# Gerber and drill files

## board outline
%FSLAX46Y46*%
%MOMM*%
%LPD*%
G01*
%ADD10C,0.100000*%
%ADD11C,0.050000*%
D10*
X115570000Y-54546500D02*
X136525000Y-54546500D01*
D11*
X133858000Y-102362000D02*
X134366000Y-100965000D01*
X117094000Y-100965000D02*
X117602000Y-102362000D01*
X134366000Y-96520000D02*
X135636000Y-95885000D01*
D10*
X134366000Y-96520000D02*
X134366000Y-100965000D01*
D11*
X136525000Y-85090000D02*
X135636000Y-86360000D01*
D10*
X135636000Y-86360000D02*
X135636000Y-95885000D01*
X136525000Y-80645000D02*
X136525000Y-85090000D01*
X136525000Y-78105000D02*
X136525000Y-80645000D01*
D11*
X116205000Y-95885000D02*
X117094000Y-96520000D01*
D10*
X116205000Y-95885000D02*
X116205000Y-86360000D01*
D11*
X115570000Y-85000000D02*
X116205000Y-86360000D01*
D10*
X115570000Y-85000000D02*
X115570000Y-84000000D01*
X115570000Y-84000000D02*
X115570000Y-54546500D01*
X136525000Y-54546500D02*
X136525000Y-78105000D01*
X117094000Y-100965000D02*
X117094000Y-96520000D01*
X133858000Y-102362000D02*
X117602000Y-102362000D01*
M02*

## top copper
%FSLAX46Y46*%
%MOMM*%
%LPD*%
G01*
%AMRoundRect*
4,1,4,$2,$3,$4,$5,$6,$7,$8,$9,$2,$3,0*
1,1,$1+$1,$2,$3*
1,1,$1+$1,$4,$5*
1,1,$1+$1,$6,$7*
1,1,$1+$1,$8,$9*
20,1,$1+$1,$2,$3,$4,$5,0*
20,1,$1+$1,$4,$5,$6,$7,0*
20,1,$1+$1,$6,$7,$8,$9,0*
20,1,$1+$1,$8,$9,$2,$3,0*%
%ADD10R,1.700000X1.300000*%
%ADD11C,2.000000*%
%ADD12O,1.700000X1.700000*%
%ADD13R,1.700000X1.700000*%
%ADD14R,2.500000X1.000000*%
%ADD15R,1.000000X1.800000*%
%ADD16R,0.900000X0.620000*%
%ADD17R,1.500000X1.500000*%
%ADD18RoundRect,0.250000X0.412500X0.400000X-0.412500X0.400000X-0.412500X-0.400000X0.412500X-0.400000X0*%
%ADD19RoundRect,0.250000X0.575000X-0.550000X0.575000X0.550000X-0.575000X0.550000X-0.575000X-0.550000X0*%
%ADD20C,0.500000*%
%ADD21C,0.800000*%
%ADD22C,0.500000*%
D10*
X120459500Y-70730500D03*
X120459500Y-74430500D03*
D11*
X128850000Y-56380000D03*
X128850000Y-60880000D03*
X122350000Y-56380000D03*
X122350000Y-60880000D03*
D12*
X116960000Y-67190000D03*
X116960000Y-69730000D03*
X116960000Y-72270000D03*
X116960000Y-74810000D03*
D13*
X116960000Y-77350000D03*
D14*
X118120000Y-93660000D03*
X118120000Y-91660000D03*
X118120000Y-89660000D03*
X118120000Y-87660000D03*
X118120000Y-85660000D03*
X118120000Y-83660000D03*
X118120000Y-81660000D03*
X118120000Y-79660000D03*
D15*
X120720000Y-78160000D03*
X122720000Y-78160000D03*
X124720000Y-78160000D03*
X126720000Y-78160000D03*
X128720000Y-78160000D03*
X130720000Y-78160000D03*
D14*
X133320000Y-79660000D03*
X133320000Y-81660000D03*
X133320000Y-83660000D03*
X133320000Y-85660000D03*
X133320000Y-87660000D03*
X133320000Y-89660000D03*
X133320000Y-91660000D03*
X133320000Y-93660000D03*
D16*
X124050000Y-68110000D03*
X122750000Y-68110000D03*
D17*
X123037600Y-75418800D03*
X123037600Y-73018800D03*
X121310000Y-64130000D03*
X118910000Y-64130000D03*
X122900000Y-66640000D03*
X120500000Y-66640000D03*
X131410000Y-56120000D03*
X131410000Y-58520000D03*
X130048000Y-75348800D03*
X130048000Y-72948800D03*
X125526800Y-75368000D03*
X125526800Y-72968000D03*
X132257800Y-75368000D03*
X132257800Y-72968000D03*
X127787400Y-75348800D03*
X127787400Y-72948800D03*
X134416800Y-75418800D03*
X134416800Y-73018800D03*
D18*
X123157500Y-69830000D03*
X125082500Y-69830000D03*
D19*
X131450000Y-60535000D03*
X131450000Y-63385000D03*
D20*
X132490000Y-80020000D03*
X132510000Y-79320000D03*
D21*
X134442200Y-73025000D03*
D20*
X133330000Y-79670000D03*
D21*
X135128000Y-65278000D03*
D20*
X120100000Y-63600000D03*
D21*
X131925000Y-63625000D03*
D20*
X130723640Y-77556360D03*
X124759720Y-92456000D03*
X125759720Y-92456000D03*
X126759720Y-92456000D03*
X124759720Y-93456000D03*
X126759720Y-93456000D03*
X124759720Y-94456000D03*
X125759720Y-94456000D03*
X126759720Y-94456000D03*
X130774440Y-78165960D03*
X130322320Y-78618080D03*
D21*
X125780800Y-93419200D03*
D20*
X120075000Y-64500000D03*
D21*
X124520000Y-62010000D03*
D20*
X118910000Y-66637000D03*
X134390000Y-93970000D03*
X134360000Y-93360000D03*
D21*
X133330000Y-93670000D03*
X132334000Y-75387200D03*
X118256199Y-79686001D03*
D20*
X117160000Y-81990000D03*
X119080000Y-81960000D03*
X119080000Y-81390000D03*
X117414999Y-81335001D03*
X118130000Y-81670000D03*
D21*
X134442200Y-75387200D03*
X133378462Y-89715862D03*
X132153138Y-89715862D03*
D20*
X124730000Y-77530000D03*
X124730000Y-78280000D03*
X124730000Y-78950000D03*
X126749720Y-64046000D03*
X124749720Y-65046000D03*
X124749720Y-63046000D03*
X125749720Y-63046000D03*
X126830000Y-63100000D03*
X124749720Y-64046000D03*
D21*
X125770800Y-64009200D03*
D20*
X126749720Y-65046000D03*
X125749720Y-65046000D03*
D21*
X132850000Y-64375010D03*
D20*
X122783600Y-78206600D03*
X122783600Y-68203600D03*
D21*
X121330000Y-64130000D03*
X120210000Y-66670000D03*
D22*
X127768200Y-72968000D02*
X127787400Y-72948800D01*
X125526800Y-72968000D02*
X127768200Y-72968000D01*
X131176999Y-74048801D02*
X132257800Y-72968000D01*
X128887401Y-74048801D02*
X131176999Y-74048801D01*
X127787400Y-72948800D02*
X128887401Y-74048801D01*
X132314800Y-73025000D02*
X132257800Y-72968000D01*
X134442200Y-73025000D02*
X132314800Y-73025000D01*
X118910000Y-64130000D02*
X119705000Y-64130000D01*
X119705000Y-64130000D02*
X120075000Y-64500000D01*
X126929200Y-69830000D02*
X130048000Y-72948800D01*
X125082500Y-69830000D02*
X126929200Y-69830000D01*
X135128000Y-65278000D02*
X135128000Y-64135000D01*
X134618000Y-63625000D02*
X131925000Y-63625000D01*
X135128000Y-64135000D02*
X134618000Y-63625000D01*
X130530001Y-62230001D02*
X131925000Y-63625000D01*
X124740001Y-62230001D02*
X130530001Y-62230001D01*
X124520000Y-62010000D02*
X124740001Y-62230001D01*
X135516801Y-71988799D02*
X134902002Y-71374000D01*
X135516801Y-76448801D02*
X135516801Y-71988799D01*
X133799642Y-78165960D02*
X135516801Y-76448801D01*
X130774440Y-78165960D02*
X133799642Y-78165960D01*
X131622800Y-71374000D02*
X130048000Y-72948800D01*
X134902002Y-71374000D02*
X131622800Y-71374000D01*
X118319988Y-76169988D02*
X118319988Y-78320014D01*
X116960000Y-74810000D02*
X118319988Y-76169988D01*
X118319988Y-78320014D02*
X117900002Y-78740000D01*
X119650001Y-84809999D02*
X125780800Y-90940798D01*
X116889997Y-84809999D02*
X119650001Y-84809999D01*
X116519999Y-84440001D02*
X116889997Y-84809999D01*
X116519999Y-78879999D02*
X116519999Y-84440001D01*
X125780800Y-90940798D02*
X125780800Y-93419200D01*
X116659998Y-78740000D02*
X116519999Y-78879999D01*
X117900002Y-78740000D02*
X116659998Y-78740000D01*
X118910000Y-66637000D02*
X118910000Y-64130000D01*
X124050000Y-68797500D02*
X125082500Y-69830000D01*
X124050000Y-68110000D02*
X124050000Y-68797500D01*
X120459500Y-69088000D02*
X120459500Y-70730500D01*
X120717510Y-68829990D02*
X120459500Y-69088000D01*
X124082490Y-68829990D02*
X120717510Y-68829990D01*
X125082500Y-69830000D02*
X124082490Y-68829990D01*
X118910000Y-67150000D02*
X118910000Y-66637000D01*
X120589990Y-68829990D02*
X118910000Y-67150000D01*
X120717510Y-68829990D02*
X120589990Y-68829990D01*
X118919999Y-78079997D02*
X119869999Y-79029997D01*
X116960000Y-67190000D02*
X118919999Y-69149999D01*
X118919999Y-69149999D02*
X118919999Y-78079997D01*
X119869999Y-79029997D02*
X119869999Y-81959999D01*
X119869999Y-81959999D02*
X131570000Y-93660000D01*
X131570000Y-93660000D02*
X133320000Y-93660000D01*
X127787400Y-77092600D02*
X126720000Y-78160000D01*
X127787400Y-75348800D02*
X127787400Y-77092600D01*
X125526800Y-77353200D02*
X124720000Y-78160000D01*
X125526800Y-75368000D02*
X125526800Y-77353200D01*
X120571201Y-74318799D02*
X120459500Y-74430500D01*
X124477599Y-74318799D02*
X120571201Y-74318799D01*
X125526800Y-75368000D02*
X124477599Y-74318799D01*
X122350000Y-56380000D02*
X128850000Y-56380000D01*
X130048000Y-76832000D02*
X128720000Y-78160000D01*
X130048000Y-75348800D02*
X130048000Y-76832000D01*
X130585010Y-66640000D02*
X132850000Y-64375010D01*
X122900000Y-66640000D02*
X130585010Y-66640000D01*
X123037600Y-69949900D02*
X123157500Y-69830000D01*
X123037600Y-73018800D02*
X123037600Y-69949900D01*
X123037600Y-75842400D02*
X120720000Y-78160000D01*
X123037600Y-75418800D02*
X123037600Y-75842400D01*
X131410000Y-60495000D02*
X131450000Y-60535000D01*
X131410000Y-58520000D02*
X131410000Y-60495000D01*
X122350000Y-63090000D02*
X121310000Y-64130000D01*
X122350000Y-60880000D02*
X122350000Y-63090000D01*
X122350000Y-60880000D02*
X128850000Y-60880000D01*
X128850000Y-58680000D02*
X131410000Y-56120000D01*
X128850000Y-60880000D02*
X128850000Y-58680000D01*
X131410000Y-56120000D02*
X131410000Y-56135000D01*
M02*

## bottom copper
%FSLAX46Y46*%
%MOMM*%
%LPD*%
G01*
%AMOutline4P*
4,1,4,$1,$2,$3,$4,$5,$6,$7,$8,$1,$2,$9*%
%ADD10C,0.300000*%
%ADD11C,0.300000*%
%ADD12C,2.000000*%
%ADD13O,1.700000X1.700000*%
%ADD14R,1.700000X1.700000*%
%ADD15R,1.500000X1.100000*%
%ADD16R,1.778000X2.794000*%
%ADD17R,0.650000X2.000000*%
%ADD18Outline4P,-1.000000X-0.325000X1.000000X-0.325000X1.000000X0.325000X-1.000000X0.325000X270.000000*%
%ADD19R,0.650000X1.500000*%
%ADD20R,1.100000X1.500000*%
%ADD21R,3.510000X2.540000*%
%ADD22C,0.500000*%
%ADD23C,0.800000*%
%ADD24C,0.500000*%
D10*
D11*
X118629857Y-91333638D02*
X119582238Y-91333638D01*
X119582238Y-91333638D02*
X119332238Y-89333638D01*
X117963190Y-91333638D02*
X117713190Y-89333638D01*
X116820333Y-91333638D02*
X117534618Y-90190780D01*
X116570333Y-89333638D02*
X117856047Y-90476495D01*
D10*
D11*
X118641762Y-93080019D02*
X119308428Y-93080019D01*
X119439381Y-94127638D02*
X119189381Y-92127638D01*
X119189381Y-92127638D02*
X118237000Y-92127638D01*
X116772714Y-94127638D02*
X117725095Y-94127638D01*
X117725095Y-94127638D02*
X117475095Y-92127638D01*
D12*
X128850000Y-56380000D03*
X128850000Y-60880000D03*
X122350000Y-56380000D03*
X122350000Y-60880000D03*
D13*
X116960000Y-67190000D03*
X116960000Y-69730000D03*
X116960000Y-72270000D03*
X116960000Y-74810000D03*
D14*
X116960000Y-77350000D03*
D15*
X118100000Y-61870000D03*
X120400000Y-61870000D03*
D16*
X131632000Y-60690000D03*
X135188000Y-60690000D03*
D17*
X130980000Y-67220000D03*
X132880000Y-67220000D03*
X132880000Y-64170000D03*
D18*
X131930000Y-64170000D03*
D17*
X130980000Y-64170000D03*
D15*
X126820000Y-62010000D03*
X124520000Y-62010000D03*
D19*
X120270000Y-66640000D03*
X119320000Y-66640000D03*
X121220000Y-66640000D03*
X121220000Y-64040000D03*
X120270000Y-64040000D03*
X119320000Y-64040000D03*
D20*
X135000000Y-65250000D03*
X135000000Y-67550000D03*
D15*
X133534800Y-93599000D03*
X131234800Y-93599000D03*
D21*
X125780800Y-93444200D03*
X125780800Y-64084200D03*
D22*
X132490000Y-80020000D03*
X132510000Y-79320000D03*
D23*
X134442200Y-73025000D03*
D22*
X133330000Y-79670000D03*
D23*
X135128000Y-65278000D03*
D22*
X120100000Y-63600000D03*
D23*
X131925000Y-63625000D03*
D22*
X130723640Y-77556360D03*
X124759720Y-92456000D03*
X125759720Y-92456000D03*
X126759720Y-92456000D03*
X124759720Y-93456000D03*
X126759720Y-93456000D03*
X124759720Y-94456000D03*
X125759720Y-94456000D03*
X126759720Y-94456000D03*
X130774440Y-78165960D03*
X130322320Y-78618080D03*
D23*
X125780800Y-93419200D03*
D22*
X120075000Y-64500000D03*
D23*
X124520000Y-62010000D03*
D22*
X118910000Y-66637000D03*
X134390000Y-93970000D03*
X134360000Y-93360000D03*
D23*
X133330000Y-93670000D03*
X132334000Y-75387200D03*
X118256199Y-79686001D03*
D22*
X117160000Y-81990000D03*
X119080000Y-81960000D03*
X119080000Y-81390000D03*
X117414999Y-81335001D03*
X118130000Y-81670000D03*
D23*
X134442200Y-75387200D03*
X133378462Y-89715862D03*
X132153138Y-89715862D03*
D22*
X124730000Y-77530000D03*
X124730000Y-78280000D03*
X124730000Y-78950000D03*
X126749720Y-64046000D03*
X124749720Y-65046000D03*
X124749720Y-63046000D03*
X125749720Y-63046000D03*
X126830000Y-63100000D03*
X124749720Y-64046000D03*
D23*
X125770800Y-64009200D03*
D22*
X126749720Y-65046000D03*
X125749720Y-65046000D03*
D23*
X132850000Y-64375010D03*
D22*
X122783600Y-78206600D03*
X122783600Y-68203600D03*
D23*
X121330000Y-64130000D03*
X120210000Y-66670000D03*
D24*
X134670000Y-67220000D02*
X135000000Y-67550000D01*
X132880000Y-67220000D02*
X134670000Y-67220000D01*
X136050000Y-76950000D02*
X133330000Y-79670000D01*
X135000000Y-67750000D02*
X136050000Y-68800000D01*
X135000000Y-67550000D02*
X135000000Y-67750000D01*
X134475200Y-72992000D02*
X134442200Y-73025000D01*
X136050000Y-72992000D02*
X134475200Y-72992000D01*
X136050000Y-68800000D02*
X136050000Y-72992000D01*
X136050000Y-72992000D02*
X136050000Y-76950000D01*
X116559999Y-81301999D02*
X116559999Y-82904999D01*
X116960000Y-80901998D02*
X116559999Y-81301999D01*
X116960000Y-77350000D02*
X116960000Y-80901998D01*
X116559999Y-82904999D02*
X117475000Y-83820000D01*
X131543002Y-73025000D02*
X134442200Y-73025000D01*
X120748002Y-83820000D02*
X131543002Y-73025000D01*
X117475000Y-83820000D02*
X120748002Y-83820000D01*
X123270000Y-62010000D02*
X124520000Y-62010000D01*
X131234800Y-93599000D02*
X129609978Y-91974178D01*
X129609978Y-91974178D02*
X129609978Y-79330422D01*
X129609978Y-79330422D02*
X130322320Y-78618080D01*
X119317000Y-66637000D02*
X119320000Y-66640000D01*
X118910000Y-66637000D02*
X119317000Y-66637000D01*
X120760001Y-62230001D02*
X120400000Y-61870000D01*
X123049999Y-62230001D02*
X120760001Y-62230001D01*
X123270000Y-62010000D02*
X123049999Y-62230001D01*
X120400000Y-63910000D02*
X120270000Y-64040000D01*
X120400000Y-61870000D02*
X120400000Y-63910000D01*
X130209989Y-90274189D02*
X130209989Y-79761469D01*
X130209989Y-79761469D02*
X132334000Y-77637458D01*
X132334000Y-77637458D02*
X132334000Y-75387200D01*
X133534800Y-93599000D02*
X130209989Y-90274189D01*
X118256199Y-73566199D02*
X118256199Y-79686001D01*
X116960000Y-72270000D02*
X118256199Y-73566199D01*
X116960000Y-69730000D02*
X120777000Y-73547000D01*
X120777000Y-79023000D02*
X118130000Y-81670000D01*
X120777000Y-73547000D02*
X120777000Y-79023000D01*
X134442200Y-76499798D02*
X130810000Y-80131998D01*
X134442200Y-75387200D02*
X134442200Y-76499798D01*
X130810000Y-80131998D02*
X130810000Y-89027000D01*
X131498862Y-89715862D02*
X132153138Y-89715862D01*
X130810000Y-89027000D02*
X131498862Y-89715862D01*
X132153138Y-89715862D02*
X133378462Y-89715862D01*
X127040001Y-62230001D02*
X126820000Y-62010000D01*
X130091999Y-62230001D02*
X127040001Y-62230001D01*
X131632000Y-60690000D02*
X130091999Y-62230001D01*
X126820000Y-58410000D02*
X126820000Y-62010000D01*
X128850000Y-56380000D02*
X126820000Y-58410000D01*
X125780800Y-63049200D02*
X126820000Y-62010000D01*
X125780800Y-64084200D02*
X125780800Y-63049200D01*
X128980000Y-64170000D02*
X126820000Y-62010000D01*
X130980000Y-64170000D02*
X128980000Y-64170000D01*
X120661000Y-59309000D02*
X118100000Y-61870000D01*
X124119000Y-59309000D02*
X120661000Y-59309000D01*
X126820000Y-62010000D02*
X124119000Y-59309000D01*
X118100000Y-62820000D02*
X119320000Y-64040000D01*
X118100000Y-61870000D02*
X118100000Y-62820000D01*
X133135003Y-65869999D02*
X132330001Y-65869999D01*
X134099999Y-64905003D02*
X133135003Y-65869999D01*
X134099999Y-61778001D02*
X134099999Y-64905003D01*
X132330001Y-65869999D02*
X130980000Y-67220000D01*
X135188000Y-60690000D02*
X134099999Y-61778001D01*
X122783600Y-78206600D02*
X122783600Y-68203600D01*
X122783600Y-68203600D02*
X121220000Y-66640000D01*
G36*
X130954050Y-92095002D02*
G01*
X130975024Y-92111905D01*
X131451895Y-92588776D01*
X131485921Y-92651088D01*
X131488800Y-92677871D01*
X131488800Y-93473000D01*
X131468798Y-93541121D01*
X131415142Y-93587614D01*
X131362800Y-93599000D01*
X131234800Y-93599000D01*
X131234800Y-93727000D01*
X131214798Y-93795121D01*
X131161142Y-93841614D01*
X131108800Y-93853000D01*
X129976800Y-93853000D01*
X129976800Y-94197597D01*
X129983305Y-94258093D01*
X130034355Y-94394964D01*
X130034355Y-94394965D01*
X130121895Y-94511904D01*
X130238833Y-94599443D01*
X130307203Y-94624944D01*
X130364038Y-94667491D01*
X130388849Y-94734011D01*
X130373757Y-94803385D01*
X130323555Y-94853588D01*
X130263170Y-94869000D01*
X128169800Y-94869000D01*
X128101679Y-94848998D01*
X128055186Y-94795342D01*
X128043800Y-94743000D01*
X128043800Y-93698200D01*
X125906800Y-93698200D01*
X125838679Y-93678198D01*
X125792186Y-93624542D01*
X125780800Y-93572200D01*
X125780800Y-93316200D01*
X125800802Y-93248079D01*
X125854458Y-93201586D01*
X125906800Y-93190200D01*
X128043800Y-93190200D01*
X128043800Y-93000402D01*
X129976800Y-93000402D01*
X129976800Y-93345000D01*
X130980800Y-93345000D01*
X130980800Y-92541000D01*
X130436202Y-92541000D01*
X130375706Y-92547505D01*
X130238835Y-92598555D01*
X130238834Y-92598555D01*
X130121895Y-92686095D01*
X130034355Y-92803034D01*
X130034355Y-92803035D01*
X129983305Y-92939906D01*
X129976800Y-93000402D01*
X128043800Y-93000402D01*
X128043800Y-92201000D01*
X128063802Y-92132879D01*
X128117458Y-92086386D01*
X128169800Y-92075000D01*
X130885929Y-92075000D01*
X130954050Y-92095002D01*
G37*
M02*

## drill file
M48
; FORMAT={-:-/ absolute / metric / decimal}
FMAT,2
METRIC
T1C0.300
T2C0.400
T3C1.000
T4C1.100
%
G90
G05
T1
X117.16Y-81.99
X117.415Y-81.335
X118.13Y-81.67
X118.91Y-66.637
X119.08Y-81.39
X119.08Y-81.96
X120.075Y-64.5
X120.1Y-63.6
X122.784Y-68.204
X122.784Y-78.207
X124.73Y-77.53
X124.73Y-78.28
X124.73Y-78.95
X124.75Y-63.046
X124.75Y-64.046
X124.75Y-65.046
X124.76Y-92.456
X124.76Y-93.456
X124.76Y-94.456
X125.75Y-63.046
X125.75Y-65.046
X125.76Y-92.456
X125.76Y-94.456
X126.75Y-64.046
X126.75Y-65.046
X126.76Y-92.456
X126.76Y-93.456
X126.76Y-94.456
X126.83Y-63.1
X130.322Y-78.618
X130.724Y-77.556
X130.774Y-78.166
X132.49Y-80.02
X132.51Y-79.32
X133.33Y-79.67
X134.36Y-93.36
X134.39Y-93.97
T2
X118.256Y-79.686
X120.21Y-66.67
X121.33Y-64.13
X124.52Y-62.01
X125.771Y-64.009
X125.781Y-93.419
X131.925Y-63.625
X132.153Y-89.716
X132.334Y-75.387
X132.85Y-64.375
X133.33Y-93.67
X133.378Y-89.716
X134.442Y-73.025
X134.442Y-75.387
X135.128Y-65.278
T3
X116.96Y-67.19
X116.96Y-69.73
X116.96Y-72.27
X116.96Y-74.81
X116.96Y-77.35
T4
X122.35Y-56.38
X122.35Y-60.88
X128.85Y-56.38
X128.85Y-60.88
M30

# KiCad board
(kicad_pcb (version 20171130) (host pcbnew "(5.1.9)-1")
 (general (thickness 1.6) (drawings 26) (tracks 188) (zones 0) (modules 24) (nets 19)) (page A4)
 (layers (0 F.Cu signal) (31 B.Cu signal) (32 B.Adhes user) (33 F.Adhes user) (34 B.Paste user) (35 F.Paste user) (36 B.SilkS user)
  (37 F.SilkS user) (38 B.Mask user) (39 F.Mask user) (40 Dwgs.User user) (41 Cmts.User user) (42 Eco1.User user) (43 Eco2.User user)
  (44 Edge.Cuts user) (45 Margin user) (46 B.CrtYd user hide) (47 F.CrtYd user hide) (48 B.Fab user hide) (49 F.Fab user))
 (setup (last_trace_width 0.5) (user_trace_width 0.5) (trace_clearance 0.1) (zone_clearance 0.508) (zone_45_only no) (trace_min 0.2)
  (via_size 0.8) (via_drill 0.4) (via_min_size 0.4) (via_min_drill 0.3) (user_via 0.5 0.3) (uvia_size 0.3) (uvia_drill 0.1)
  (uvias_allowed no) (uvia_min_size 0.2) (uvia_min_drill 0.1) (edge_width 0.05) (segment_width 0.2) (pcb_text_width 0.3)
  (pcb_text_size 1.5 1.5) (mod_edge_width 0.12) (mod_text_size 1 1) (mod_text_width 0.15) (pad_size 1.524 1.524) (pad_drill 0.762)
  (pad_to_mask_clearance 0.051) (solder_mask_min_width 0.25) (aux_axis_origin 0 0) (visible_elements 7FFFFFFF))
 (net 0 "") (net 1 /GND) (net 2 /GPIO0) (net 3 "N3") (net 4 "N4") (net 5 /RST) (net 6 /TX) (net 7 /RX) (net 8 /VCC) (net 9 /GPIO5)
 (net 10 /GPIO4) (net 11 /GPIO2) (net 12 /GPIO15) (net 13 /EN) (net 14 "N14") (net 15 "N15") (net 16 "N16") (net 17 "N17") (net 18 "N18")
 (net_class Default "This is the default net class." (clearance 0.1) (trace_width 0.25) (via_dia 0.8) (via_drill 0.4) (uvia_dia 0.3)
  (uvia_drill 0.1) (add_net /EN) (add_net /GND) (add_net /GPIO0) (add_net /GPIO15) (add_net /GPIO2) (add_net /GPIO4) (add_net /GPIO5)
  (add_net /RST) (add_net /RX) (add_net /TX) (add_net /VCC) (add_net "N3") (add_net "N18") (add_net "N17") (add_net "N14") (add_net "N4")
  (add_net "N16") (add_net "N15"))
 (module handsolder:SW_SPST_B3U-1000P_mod (layer F.Cu) (at 120.4595 72.5805 90)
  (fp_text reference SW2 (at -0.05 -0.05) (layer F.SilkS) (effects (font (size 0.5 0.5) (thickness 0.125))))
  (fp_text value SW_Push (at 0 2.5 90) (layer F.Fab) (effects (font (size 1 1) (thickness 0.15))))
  (pad 2 smd rect (at 1.85 0 90) (size 1.3 1.7) (layers F.Cu F.Paste F.Mask) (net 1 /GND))
  (pad 1 smd rect (at -1.85 0 90) (size 1.3 1.7) (layers F.Cu F.Paste F.Mask) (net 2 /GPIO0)))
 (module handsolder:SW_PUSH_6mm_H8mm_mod (layer F.Cu) (at 122.35 56.38)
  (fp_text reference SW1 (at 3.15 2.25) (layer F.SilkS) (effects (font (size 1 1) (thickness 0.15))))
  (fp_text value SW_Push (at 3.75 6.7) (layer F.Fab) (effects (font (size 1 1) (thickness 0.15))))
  (pad 1 thru_hole circle (at 6.5 0 90) (size 2 2) (drill 1.1) (layers *.Cu *.Mask) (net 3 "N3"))
  (pad 2 thru_hole circle (at 6.5 4.5 90) (size 2 2) (drill 1.1) (layers *.Cu *.Mask) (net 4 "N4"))
  (pad 1 thru_hole circle (at 0 0 90) (size 2 2) (drill 1.1) (layers *.Cu *.Mask) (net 3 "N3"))
  (pad 2 thru_hole circle (at 0 4.5 90) (size 2 2) (drill 1.1) (layers *.Cu *.Mask) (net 4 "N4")))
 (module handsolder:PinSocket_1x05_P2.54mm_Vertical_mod (layer F.Cu) (at 116.96 77.35 180)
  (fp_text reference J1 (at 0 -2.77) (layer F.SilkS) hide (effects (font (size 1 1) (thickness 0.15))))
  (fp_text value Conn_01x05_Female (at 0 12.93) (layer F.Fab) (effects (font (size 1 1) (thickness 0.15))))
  (pad 5 thru_hole oval (at 0 10.16 180) (size 1.7 1.7) (drill 1) (layers *.Cu *.Mask) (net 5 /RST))
  (pad 4 thru_hole oval (at 0 7.62 180) (size 1.7 1.7) (drill 1) (layers *.Cu *.Mask) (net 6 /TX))
  (pad 3 thru_hole oval (at 0 5.08 180) (size 1.7 1.7) (drill 1) (layers *.Cu *.Mask) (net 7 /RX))
  (pad 2 thru_hole oval (at 0 2.54 180) (size 1.7 1.7) (drill 1) (layers *.Cu *.Mask) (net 1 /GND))
  (pad 1 thru_hole rect (at 0 0 180) (size 1.7 1.7) (drill 1) (layers *.Cu *.Mask) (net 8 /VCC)))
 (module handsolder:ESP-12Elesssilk (layer F.Cu) (at 125.72 90.16 180)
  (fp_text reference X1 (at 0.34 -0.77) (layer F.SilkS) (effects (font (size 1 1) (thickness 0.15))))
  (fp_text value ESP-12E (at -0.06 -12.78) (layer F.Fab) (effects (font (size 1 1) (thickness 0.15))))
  (pad 22 smd rect (at 7.6 -3.5 180) (size 2.5 1) (layers F.Cu F.Paste F.Mask))
  (pad 21 smd rect (at 7.6 -1.5 180) (size 2.5 1) (layers F.Cu F.Paste F.Mask))
  (pad 20 smd rect (at 7.6 0.5 180) (size 2.5 1) (layers F.Cu F.Paste F.Mask))
  (pad 19 smd rect (at 7.6 2.5 180) (size 2.5 1) (layers F.Cu F.Paste F.Mask))
  (pad 18 smd rect (at 7.6 4.5 180) (size 2.5 1) (layers F.Cu F.Paste F.Mask))
  (pad 17 smd rect (at 7.6 6.5 180) (size 2.5 1) (layers F.Cu F.Paste F.Mask))
  (pad 16 smd rect (at 7.6 8.5 180) (size 2.5 1) (layers F.Cu F.Paste F.Mask) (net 6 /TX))
  (pad 15 smd rect (at 7.6 10.5 180) (size 2.5 1) (layers F.Cu F.Paste F.Mask) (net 7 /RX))
  (pad 14 smd rect (at 5 12 180) (size 1 1.8) (layers F.Cu F.Paste F.Mask) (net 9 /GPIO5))
  (pad 13 smd rect (at 3 12 180) (size 1 1.8) (layers F.Cu F.Paste F.Mask) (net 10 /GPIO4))
  (pad 12 smd rect (at 1 12 180) (size 1 1.8) (layers F.Cu F.Paste F.Mask) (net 2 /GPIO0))
  (pad 11 smd rect (at -1 12 180) (size 1 1.8) (layers F.Cu F.Paste F.Mask) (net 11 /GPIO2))
  (pad 10 smd rect (at -3 12 180) (size 1 1.8) (layers F.Cu F.Paste F.Mask) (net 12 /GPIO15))
  (pad 9 smd rect (at -5 12 180) (size 1 1.8) (layers F.Cu F.Paste F.Mask) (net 1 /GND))
  (pad 8 smd rect (at -7.6 10.5 180) (size 2.5 1) (layers F.Cu F.Paste F.Mask) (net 8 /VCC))
  (pad 7 smd rect (at -7.6 8.5 180) (size 2.5 1) (layers F.Cu F.Paste F.Mask))
  (pad 6 smd rect (at -7.6 6.5 180) (size 2.5 1) (layers F.Cu F.Paste F.Mask))
  (pad 5 smd rect (at -7.6 4.5 180) (size 2.5 1) (layers F.Cu F.Paste F.Mask))
  (pad 4 smd rect (at -7.6 2.5 180) (size 2.5 1) (layers F.Cu F.Paste F.Mask))
  (pad 3 smd rect (at -7.6 0.5 180) (size 2.5 1) (layers F.Cu F.Paste F.Mask) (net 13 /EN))
  (pad 2 smd rect (at -7.6 -1.5 180) (size 2.5 1) (layers F.Cu F.Paste F.Mask))
  (pad 1 smd rect (at -7.6 -3.5 180) (size 2.5 1) (layers F.Cu F.Paste F.Mask) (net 5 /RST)))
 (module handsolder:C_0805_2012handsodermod (layer B.Cu) (at 119.25 61.87 180)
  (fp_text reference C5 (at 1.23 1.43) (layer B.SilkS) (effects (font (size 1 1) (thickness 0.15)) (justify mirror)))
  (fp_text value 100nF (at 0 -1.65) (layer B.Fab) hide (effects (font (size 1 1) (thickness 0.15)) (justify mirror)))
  (pad 2 smd rect (at 1.15 0 180) (size 1.5 1.1) (layers B.Cu B.Paste B.Mask) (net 3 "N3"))
  (pad 1 smd rect (at -1.15 0 180) (size 1.5 1.1) (layers B.Cu B.Paste B.Mask) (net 1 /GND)))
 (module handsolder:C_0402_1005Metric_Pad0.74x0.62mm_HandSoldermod (layer F.Cu) (at 123.4 68.11)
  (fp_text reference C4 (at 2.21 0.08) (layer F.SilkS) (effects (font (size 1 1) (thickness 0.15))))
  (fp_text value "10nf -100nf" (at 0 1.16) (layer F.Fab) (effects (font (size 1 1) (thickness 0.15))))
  (pad 2 smd rect (at 0.65 0) (size 0.9 0.62) (layers F.Cu F.Paste F.Mask) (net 1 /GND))
  (pad 1 smd rect (at -0.65 0) (size 0.9 0.62) (layers F.Cu F.Paste F.Mask) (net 10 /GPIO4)))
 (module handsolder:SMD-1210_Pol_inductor (layer B.Cu) (at 133.41 60.69)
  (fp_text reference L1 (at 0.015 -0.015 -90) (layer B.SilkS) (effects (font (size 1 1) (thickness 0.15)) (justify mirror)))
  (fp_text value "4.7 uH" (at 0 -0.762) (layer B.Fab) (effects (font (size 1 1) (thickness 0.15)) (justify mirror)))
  (pad 1 smd rect (at -1.778 0) (size 1.778 2.794) (layers B.Cu B.Paste B.Mask) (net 3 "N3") (zone_connect 2))
  (pad 2 smd rect (at 1.778 0) (size 1.778 2.794) (layers B.Cu B.Paste B.Mask) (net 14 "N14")))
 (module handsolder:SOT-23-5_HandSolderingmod (layer B.Cu) (at 131.93 65.72 270)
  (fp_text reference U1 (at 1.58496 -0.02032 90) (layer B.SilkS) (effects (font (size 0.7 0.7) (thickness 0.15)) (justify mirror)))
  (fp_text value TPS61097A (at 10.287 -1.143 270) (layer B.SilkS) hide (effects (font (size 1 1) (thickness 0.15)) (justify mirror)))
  (pad 5 smd rect (at 1.5 0.95 270) (size 2 0.65) (layers B.Cu B.Paste B.Mask) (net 14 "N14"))
  (pad 4 smd rect (at 1.5 -0.95 270) (size 2 0.65) (layers B.Cu B.Paste B.Mask) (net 8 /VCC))
  (pad 3 smd rect (at -1.55 -0.95 270) (size 2 0.65) (layers B.Cu B.Paste B.Mask) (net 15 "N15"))
  (pad 2 smd trapezoid (at -1.55 0 270) (size 2 0.65) (layers B.Cu B.Paste B.Mask) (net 1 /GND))
  (pad 1 smd rect (at -1.55 0.95 270) (size 2 0.65) (layers B.Cu B.Paste B.Mask) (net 3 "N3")))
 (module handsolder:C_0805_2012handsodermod (layer B.Cu) (at 125.67 62.01)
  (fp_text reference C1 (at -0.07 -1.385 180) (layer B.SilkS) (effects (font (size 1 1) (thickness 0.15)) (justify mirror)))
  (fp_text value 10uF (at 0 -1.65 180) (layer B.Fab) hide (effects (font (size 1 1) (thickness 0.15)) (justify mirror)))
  (pad 2 smd rect (at 1.15 0) (size 1.5 1.1) (layers B.Cu B.Paste B.Mask) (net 3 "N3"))
  (pad 1 smd rect (at -1.15 0) (size 1.5 1.1) (layers B.Cu B.Paste B.Mask) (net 1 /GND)))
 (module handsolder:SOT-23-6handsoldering (layer B.Cu) (at 120.27 65.34 270)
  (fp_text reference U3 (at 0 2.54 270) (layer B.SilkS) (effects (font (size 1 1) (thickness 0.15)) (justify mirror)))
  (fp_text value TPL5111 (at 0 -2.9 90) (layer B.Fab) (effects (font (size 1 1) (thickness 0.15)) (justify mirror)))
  (pad 5 smd rect (at 1.3 0 270) (size 1.5 0.65) (layers B.Cu B.Paste B.Mask) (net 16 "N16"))
  (pad 6 smd rect (at 1.3 0.95 270) (size 1.5 0.65) (layers B.Cu B.Paste B.Mask) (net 1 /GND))
  (pad 4 smd rect (at 1.3 -0.95 270) (size 1.5 0.65) (layers B.Cu B.Paste B.Mask) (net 10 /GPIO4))
  (pad 3 smd rect (at -1.3 -0.95 270) (size 1.5 0.65) (layers B.Cu B.Paste B.Mask) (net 4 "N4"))
  (pad 2 smd rect (at -1.3 0 270) (size 1.5 0.65) (layers B.Cu B.Paste B.Mask) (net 1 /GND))
  (pad 1 smd rect (at -1.3 0.95 270) (size 1.5 0.65) (layers B.Cu B.Paste B.Mask) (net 3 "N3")))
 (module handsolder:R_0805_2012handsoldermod (layer F.Cu) (at 123.0376 74.2188 270)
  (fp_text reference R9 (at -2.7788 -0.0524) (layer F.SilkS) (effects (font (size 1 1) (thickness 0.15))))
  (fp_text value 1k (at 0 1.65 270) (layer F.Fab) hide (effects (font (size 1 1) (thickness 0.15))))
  (pad 2 smd rect (at 1.2 0 270) (size 1.5 1.5) (layers F.Cu F.Paste F.Mask) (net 9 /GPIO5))
  (pad 1 smd rect (at -1.2 0 270) (size 1.5 1.5) (layers F.Cu F.Paste F.Mask) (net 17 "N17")))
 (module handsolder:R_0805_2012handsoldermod (layer F.Cu) (at 120.11 64.13)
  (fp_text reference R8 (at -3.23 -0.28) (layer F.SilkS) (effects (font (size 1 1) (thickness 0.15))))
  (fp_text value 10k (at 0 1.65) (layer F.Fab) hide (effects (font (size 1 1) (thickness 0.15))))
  (pad 2 smd rect (at 1.2 0) (size 1.5 1.5) (layers F.Cu F.Paste F.Mask) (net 4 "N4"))
  (pad 1 smd rect (at -1.2 0) (size 1.5 1.5) (layers F.Cu F.Paste F.Mask) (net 1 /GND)))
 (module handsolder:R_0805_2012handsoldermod (layer F.Cu) (at 121.7 66.64)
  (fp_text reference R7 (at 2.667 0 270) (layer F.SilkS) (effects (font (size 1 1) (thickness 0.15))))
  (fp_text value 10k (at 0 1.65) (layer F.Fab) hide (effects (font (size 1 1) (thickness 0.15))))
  (pad 2 smd rect (at 1.2 0) (size 1.5 1.5) (layers F.Cu F.Paste F.Mask) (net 15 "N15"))
  (pad 1 smd rect (at -1.2 0) (size 1.5 1.5) (layers F.Cu F.Paste F.Mask) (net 16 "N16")))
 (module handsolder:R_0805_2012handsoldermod (layer F.Cu) (at 131.41 57.32 90)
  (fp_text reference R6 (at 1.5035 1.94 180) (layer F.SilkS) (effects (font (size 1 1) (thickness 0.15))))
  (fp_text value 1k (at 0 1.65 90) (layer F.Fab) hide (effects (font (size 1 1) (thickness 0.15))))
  (pad 2 smd rect (at 1.2 0 90) (size 1.5 1.5) (layers F.Cu F.Paste F.Mask) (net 4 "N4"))
  (pad 1 smd rect (at -1.2 0 90) (size 1.5 1.5) (layers F.Cu F.Paste F.Mask) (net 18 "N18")))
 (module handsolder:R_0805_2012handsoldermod (layer F.Cu) (at 130.048 74.1488 270)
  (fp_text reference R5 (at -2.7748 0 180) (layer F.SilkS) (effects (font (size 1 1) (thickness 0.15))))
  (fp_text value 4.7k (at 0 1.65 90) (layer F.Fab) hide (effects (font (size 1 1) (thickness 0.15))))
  (pad 2 smd rect (at 1.2 0 270) (size 1.5 1.5) (layers F.Cu F.Paste F.Mask) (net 12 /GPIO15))
  (pad 1 smd rect (at -1.2 0 270) (size 1.5 1.5) (layers F.Cu F.Paste F.Mask) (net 1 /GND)))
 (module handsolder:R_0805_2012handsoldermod (layer F.Cu) (at 125.5268 74.168 270)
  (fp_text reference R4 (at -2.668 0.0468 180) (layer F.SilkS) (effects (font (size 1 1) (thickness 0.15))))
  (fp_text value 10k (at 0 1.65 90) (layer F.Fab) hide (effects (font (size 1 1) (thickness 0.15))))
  (pad 2 smd rect (at 1.2 0 270) (size 1.5 1.5) (layers F.Cu F.Paste F.Mask) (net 2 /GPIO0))
  (pad 1 smd rect (at -1.2 0 270) (size 1.5 1.5) (layers F.Cu F.Paste F.Mask) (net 8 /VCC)))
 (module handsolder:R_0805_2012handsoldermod (layer F.Cu) (at 132.2578 74.168 270)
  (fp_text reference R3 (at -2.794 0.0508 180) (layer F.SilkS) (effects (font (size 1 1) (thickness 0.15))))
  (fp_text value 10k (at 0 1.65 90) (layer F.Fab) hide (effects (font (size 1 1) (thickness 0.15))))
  (pad 2 smd rect (at 1.2 0 270) (size 1.5 1.5) (layers F.Cu F.Paste F.Mask) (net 5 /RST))
  (pad 1 smd rect (at -1.2 0 270) (size 1.5 1.5) (layers F.Cu F.Paste F.Mask) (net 8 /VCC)))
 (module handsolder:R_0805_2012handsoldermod (layer F.Cu) (at 127.7874 74.1488 270)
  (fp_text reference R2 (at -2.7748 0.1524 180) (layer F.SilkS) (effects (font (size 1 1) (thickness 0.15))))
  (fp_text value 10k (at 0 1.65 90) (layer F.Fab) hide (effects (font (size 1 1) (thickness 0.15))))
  (pad 2 smd rect (at 1.2 0 270) (size 1.5 1.5) (layers F.Cu F.Paste F.Mask) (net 11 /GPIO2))
  (pad 1 smd rect (at -1.2 0 270) (size 1.5 1.5) (layers F.Cu F.Paste F.Mask) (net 8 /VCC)))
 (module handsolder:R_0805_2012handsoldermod (layer F.Cu) (at 134.4168 74.2188 270)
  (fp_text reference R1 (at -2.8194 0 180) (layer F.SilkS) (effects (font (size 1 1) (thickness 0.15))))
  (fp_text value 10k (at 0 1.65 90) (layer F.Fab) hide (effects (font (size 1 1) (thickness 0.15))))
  (pad 2 smd rect (at 1.2 0 270) (size 1.5 1.5) (layers F.Cu F.Paste F.Mask) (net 13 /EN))
  (pad 1 smd rect (at -1.2 0 270) (size 1.5 1.5) (layers F.Cu F.Paste F.Mask) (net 8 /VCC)))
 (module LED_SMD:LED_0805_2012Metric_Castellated (layer F.Cu) (at 124.12 69.83 180)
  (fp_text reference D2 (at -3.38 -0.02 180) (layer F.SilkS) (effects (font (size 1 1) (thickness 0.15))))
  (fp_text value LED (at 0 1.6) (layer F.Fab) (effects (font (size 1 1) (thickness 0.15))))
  (pad 2 smd roundrect (at 0.9625 0 180) (size 1.325 1.3) (layers F.Cu F.Paste F.Mask) (roundrect_rratio 0.1923076923076923) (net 17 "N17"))
  (pad 1 smd roundrect (at -0.9625 0 180) (size 1.325 1.3) (layers F.Cu F.Paste F.Mask) (roundrect_rratio 0.1923076923076923) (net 1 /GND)))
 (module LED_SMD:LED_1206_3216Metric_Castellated (layer F.Cu) (at 131.45 61.96 90)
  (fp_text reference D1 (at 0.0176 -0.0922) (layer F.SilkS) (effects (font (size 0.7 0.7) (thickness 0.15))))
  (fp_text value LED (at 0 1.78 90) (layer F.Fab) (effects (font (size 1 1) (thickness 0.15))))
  (pad 2 smd roundrect (at 1.425 0 90) (size 1.6 1.65) (layers F.Cu F.Paste F.Mask) (roundrect_rratio 0.15625) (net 18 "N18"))
  (pad 1 smd roundrect (at -1.425 0 90) (size 1.6 1.65) (layers F.Cu F.Paste F.Mask) (roundrect_rratio 0.15625) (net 1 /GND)))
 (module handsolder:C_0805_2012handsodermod (layer B.Cu) (at 135 66.4 90)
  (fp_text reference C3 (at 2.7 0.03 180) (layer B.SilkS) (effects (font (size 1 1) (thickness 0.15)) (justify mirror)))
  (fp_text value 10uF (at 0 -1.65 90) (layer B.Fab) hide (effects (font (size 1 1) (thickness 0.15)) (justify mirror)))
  (pad 2 smd rect (at 1.15 0 90) (size 1.5 1.1) (layers B.Cu B.Paste B.Mask) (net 1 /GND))
  (pad 1 smd rect (at -1.15 0 90) (size 1.5 1.1) (layers B.Cu B.Paste B.Mask) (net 8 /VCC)))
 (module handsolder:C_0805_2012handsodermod (layer B.Cu) (at 132.3848 93.599)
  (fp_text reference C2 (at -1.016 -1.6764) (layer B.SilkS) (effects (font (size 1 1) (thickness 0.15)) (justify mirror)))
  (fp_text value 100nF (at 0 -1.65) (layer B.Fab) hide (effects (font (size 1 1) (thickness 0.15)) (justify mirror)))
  (pad 2 smd rect (at 1.15 0) (size 1.5 1.1) (layers B.Cu B.Paste B.Mask) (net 5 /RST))
  (pad 1 smd rect (at -1.15 0) (size 1.5 1.1) (layers B.Cu B.Paste B.Mask) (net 1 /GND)))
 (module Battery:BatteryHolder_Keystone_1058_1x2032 (layer B.Cu) (at 125.7808 78.7642 270)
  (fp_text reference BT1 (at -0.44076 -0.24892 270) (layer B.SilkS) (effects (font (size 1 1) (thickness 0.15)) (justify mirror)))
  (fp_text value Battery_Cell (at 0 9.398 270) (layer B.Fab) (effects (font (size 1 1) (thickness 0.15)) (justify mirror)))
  (pad 2 smd rect (at 14.68 0 270) (size 2.54 3.51) (layers B.Cu B.Paste B.Mask) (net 1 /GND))
  (pad 1 smd rect (at -14.68 0 270) (size 2.54 3.51) (layers B.Cu B.Paste B.Mask) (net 3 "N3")))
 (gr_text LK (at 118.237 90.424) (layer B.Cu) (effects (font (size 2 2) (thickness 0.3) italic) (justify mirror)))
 (gr_line (start 115.57 54.5465) (end 136.525 54.5465) (layer Edge.Cuts) (width 0.1))
 (gr_line (start 133.858 102.362) (end 134.366 100.965) (layer Edge.Cuts) (width 0.05))
 (gr_line (start 117.094 100.965) (end 117.602 102.362) (layer Edge.Cuts) (width 0.05))
 (gr_line (start 134.366 96.52) (end 135.636 95.885) (layer Edge.Cuts) (width 0.05))
 (gr_line (start 134.366 96.52) (end 134.366 100.965) (layer Edge.Cuts) (width 0.1))
 (gr_line (start 136.525 85.09) (end 135.636 86.36) (layer Edge.Cuts) (width 0.05))
 (gr_line (start 135.636 86.36) (end 135.636 95.885) (layer Edge.Cuts) (width 0.1))
 (gr_line (start 136.525 80.645) (end 136.525 85.09) (layer Edge.Cuts) (width 0.1))
 (gr_line (start 136.525 78.105) (end 136.525 80.645) (layer Edge.Cuts) (width 0.1))
 (gr_line (start 116.205 95.885) (end 117.094 96.52) (layer Edge.Cuts) (width 0.05))
 (gr_line (start 116.205 95.885) (end 116.205 86.36) (layer Edge.Cuts) (width 0.1))
 (gr_line (start 115.57 85) (end 116.205 86.36) (layer Edge.Cuts) (width 0.05))
 (gr_line (start 115.57 85) (end 115.57 84) (layer Edge.Cuts) (width 0.1))
 (gr_line (start 115.57 84) (end 115.57 54.5465) (layer Edge.Cuts) (width 0.1))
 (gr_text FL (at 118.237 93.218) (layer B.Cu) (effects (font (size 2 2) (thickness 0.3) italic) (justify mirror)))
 (gr_line (start 136.525 54.5465) (end 136.525 78.105) (layer Edge.Cuts) (width 0.1))
 (gr_line (start 117.094 100.965) (end 117.094 96.52) (layer Edge.Cuts) (width 0.1))
 (gr_line (start 133.858 102.362) (end 117.602 102.362) (layer Edge.Cuts) (width 0.1))
 (via (at 132.49 80.02) (size 0.5) (drill 0.3) (layers F.Cu B.Cu) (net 8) (status 30))
 (via (at 132.51 79.32) (size 0.5) (drill 0.3) (layers F.Cu B.Cu) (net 8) (status 30))
 (via (at 134.4422 73.025) (size 0.8) (drill 0.4) (layers F.Cu B.Cu) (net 8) (status 30))
 (via (at 133.33 79.67) (size 0.5) (drill 0.3) (layers F.Cu B.Cu) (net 8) (status 30))
 (segment (start 127.7682 72.968) (end 127.7874 72.9488) (width 0.5) (layer F.Cu) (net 8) (status 30))
 (segment (start 125.5268 72.968) (end 127.7682 72.968) (width 0.5) (layer F.Cu) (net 8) (status 30))
 (segment (start 131.176999 74.048801) (end 132.2578 72.968) (width 0.5) (layer F.Cu) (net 8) (status 20))
 (segment (start 128.887401 74.048801) (end 131.176999 74.048801) (width 0.5) (layer F.Cu) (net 8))
 (segment (start 127.7874 72.9488) (end 128.887401 74.048801) (width 0.5) (layer F.Cu) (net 8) (status 10))
 (segment (start 134.67 67.22) (end 135 67.55) (width 0.5) (layer B.Cu) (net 8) (status 30))
 (segment (start 132.88 67.22) (end 134.67 67.22) (width 0.5) (layer B.Cu) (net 8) (status 30))
 (segment (start 136.05 76.95) (end 133.33 79.67) (width 0.5) (layer B.Cu) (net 8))
 (segment (start 135 67.75) (end 136.05 68.8) (width 0.5) (layer B.Cu) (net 8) (status 10))
 (segment (start 135 67.55) (end 135 67.75) (width 0.5) (layer B.Cu) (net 8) (status 30))
 (segment (start 134.4752 72.992) (end 134.4422 73.025) (width 0.5) (layer B.Cu) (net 8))
 (segment (start 136.05 72.992) (end 134.4752 72.992) (width 0.5) (layer B.Cu) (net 8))
 (segment (start 136.05 68.8) (end 136.05 72.992) (width 0.5) (layer B.Cu) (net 8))
 (segment (start 136.05 72.992) (end 136.05 76.95) (width 0.5) (layer B.Cu) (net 8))
 (segment (start 132.3148 73.025) (end 132.2578 72.968) (width 0.5) (layer F.Cu) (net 8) (status 30))
 (segment (start 134.4422 73.025) (end 132.3148 73.025) (width 0.5) (layer F.Cu) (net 8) (status 30))
 (segment (start 116.559999 81.301999) (end 116.559999 82.904999) (width 0.5) (layer B.Cu) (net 8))
 (segment (start 116.96 80.901998) (end 116.559999 81.301999) (width 0.5) (layer B.Cu) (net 8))
 (segment (start 116.96 77.35) (end 116.96 80.901998) (width 0.5) (layer B.Cu) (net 8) (status 10))
 (segment (start 116.559999 82.904999) (end 117.475 83.82) (width 0.5) (layer B.Cu) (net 8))
 (segment (start 131.543002 73.025) (end 134.4422 73.025) (width 0.5) (layer B.Cu) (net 8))
 (segment (start 120.748002 83.82) (end 131.543002 73.025) (width 0.5) (layer B.Cu) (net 8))
 (segment (start 117.475 83.82) (end 120.748002 83.82) (width 0.5) (layer B.Cu) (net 8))
 (via (at 135.128 65.278) (size 0.8) (drill 0.4) (layers F.Cu B.Cu) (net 1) (status 30))
 (via (at 120.1 63.6) (size 0.5) (drill 0.3) (layers F.Cu B.Cu) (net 1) (status 30))
 (via (at 131.925 63.625) (size 0.8) (drill 0.4) (layers F.Cu B.Cu) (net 1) (status 30))
 (via (at 130.72364 77.55636) (size 0.5) (drill 0.3) (layers F.Cu B.Cu) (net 1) (status 30))
 (via (at 124.75972 92.456) (size 0.5) (drill 0.3) (layers F.Cu B.Cu) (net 1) (status 30))
 (via (at 125.75972 92.456) (size 0.5) (drill 0.3) (layers F.Cu B.Cu) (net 1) (status 30))
 (via (at 126.75972 92.456) (size 0.5) (drill 0.3) (layers F.Cu B.Cu) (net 1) (status 30))
 (via (at 124.75972 93.456) (size 0.5) (drill 0.3) (layers F.Cu B.Cu) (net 1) (status 30))
 (via (at 126.75972 93.456) (size 0.5) (drill 0.3) (layers F.Cu B.Cu) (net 1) (status 30))
 (via (at 124.75972 94.456) (size 0.5) (drill 0.3) (layers F.Cu B.Cu) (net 1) (status 30))
 (via (at 125.75972 94.456) (size 0.5) (drill 0.3) (layers F.Cu B.Cu) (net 1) (status 30))
 (via (at 126.75972 94.456) (size 0.5) (drill 0.3) (layers F.Cu B.Cu) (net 1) (status 30))
 (via (at 130.77444 78.16596) (size 0.5) (drill 0.3) (layers F.Cu B.Cu) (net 1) (status 30))
 (via (at 130.32232 78.61808) (size 0.5) (drill 0.3) (layers F.Cu B.Cu) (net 1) (status 30))
 (via (at 125.7808 93.4192) (size 0.8) (drill 0.4) (layers F.Cu B.Cu) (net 1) (status 30))
 (segment (start 118.91 64.13) (end 119.705 64.13) (width 0.5) (layer F.Cu) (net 1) (status 10))
 (segment (start 119.705 64.13) (end 120.075 64.5) (width 0.5) (layer F.Cu) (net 1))
 (via (at 120.075 64.5) (size 0.5) (drill 0.3) (layers F.Cu B.Cu) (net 1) (status 30))
 (segment (start 126.9292 69.83) (end 130.048 72.9488) (width 0.5) (layer F.Cu) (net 1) (status 20))
 (segment (start 125.0825 69.83) (end 126.9292 69.83) (width 0.5) (layer F.Cu) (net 1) (status 10))
 (segment (start 123.27 62.01) (end 124.52 62.01) (width 0.5) (layer B.Cu) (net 1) (status 20))
 (segment (start 135.128 65.278) (end 135.128 64.135) (width 0.5) (layer F.Cu) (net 1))
 (segment (start 134.618 63.625) (end 131.925 63.625) (width 0.5) (layer F.Cu) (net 1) (status 20))
 (segment (start 135.128 64.135) (end 134.618 63.625) (width 0.5) (layer F.Cu) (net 1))
 (segment (start 131.2348 93.599) (end 129.609978 91.974178) (width 0.5) (layer B.Cu) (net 1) (status 10))
 (segment (start 129.609978 91.974178) (end 129.609978 79.330422) (width 0.5) (layer B.Cu) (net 1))
 (segment (start 129.609978 79.330422) (end 130.32232 78.61808) (width 0.5) (layer B.Cu) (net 1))
 (via (at 124.52 62.01) (size 0.8) (drill 0.4) (layers F.Cu B.Cu) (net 1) (status 30))
 (segment (start 130.530001 62.230001) (end 131.925 63.625) (width 0.5) (layer F.Cu) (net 1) (status 20))
 (segment (start 124.740001 62.230001) (end 130.530001 62.230001) (width 0.5) (layer F.Cu) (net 1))
 (segment (start 124.52 62.01) (end 124.740001 62.230001) (width 0.5) (layer F.Cu) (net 1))
 (segment (start 135.516801 71.988799) (end 134.902002 71.374) (width 0.5) (layer F.Cu) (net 1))
 (segment (start 135.516801 76.448801) (end 135.516801 71.988799) (width 0.5) (layer F.Cu) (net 1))
 (segment (start 133.799642 78.16596) (end 135.516801 76.448801) (width 0.5) (layer F.Cu) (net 1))
 (segment (start 130.77444 78.16596) (end 133.799642 78.16596) (width 0.5) (layer F.Cu) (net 1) (status 10))
 (segment (start 131.6228 71.374) (end 130.048 72.9488) (width 0.5) (layer F.Cu) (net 1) (status 20))
 (segment (start 134.902002 71.374) (end 131.6228 71.374) (width 0.5) (layer F.Cu) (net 1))
 (segment (start 118.319988 76.169988) (end 118.319988 78.320014) (width 0.5) (layer F.Cu) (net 1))
 (segment (start 116.96 74.81) (end 118.319988 76.169988) (width 0.5) (layer F.Cu) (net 1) (status 10))
 (segment (start 118.319988 78.320014) (end 117.900002 78.74) (width 0.5) (layer F.Cu) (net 1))
 (segment (start 119.650001 84.809999) (end 125.7808 90.940798) (width 0.5) (layer F.Cu) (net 1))
 (segment (start 116.889997 84.809999) (end 119.650001 84.809999) (width 0.5) (layer F.Cu) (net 1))
 (segment (start 116.519999 84.440001) (end 116.889997 84.809999) (width 0.5) (layer F.Cu) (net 1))
 (segment (start 116.519999 78.879999) (end 116.519999 84.440001) (width 0.5) (layer F.Cu) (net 1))
 (segment (start 125.7808 90.940798) (end 125.7808 93.4192) (width 0.5) (layer F.Cu) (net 1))
 (segment (start 116.659998 78.74) (end 116.519999 78.879999) (width 0.5) (layer F.Cu) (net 1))
 (segment (start 117.900002 78.74) (end 116.659998 78.74) (width 0.5) (layer F.Cu) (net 1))
 (segment (start 118.91 66.637) (end 118.91 64.13) (width 0.5) (layer F.Cu) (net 1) (status 20))
 (via (at 118.91 66.637) (size 0.5) (drill 0.3) (layers F.Cu B.Cu) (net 1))
 (segment (start 119.317 66.637) (end 119.32 66.64) (width 0.5) (layer B.Cu) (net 1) (status 30))
 (segment (start 118.91 66.637) (end 119.317 66.637) (width 0.5) (layer B.Cu) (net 1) (status 20))
 (segment (start 124.05 68.7975) (end 125.0825 69.83) (width 0.5) (layer F.Cu) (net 1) (status 20))
 (segment (start 124.05 68.11) (end 124.05 68.7975) (width 0.5) (layer F.Cu) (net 1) (status 10))
 (segment (start 120.760001 62.230001) (end 120.4 61.87) (width 0.5) (layer B.Cu) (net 1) (status 30))
 (segment (start 123.049999 62.230001) (end 120.760001 62.230001) (width 0.5) (layer B.Cu) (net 1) (status 20))
 (segment (start 123.27 62.01) (end 123.049999 62.230001) (width 0.5) (layer B.Cu) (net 1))
 (segment (start 120.4 63.91) (end 120.27 64.04) (width 0.5) (layer B.Cu) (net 1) (status 30))
 (segment (start 120.4 61.87) (end 120.4 63.91) (width 0.5) (layer B.Cu) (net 1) (status 30))
 (segment (start 120.4595 69.088) (end 120.4595 70.7305) (width 0.5) (layer F.Cu) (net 1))
 (segment (start 120.71751 68.82999) (end 120.4595 69.088) (width 0.5) (layer F.Cu) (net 1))
 (segment (start 124.08249 68.82999) (end 120.71751 68.82999) (width 0.5) (layer F.Cu) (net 1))
 (segment (start 125.0825 69.83) (end 124.08249 68.82999) (width 0.5) (layer F.Cu) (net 1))
 (segment (start 118.91 67.15) (end 118.91 66.637) (width 0.5) (layer F.Cu) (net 1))
 (segment (start 120.58999 68.82999) (end 118.91 67.15) (width 0.5) (layer F.Cu) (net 1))
 (segment (start 120.71751 68.82999) (end 120.58999 68.82999) (width 0.5) (layer F.Cu) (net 1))
 (via (at 134.39 93.97) (size 0.5) (drill 0.3) (layers F.Cu B.Cu) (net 5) (status 30))
 (via (at 134.36 93.36) (size 0.5) (drill 0.3) (layers F.Cu B.Cu) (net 5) (status 30))
 (via (at 133.33 93.67) (size 0.8) (drill 0.4) (layers F.Cu B.Cu) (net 5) (status 30))
 (via (at 132.334 75.3872) (size 0.8) (drill 0.4) (layers F.Cu B.Cu) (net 5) (status 30))
 (segment (start 130.209989 90.274189) (end 130.209989 79.761469) (width 0.5) (layer B.Cu) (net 5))
 (segment (start 130.209989 79.761469) (end 132.334 77.637458) (width 0.5) (layer B.Cu) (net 5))
 (segment (start 132.334 77.637458) (end 132.334 75.3872) (width 0.5) (layer B.Cu) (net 5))
 (segment (start 133.5348 93.599) (end 130.209989 90.274189) (width 0.5) (layer B.Cu) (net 5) (status 10))
 (segment (start 118.919999 78.079997) (end 119.869999 79.029997) (width 0.5) (layer F.Cu) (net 5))
 (segment (start 116.96 67.19) (end 118.919999 69.149999) (width 0.5) (layer F.Cu) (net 5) (status 10))
 (segment (start 118.919999 69.149999) (end 118.919999 78.079997) (width 0.5) (layer F.Cu) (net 5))
 (segment (start 119.869999 79.029997) (end 119.869999 81.959999) (width 0.5) (layer F.Cu) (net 5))
 (segment (start 119.869999 81.959999) (end 131.57 93.66) (width 0.5) (layer F.Cu) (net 5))
 (segment (start 131.57 93.66) (end 133.32 93.66) (width 0.5) (layer F.Cu) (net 5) (status 20))
 (via (at 118.256199 79.686001) (size 0.8) (drill 0.4) (layers F.Cu B.Cu) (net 7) (status 30))
 (segment (start 118.256199 73.566199) (end 118.256199 79.686001) (width 0.5) (layer B.Cu) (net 7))
 (segment (start 116.96 72.27) (end 118.256199 73.566199) (width 0.5) (layer B.Cu) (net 7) (status 10))
 (via (at 117.16 81.99) (size 0.5) (drill 0.3) (layers F.Cu B.Cu) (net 6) (status 30))
 (via (at 119.08 81.96) (size 0.5) (drill 0.3) (layers F.Cu B.Cu) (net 6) (status 30))
 (via (at 119.08 81.39) (size 0.5) (drill 0.3) (layers F.Cu B.Cu) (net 6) (status 30))
 (via (at 117.414999 81.335001) (size 0.5) (drill 0.3) (layers F.Cu B.Cu) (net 6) (status 30))
 (via (at 118.13 81.67) (size 0.5) (drill 0.3) (layers F.Cu B.Cu) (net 6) (status 30))
 (segment (start 116.96 69.73) (end 120.777 73.547) (width 0.5) (layer B.Cu) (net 6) (status 10))
 (segment (start 120.777 79.023) (end 118.13 81.67) (width 0.5) (layer B.Cu) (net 6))
 (segment (start 120.777 73.547) (end 120.777 79.023) (width 0.5) (layer B.Cu) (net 6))
 (via (at 134.4422 75.3872) (size 0.8) (drill 0.4) (layers F.Cu B.Cu) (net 13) (status 30))
 (via (at 133.378462 89.715862) (size 0.8) (drill 0.4) (layers F.Cu B.Cu) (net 13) (status 30))
 (segment (start 134.4422 76.499798) (end 130.81 80.131998) (width 0.5) (layer B.Cu) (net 13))
 (segment (start 134.4422 75.3872) (end 134.4422 76.499798) (width 0.5) (layer B.Cu) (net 13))
 (segment (start 130.81 80.131998) (end 130.81 89.027) (width 0.5) (layer B.Cu) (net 13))
 (segment (start 131.498862 89.715862) (end 132.153138 89.715862) (width 0.5) (layer B.Cu) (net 13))
 (segment (start 130.81 89.027) (end 131.498862 89.715862) (width 0.5) (layer B.Cu) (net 13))
 (segment (start 132.153138 89.715862) (end 133.378462 89.715862) (width 0.5) (layer B.Cu) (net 13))
 (via (at 132.153138 89.715862) (size 0.8) (drill 0.4) (layers F.Cu B.Cu) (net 13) (status 30))
 (segment (start 127.7874 77.0926) (end 126.72 78.16) (width 0.5) (layer F.Cu) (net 11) (status 20))
 (segment (start 127.7874 75.3488) (end 127.7874 77.0926) (width 0.5) (layer F.Cu) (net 11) (status 10))
 (via (at 124.73 77.53) (size 0.5) (drill 0.3) (layers F.Cu B.Cu) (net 2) (status 30))
 (via (at 124.73 78.28) (size 0.5) (drill 0.3) (layers F.Cu B.Cu) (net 2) (status 30))
 (via (at 124.73 78.95) (size 0.5) (drill 0.3) (layers F.Cu B.Cu) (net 2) (status 30))
 (segment (start 125.5268 77.3532) (end 124.72 78.16) (width 0.5) (layer F.Cu) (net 2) (status 20))
 (segment (start 125.5268 75.368) (end 125.5268 77.3532) (width 0.5) (layer F.Cu) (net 2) (status 10))
 (segment (start 120.571201 74.318799) (end 120.4595 74.4305) (width 0.5) (layer F.Cu) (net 2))
 (segment (start 124.477599 74.318799) (end 120.571201 74.318799) (width 0.5) (layer F.Cu) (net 2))
 (segment (start 125.5268 75.368) (end 124.477599 74.318799) (width 0.5) (layer F.Cu) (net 2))
 (via (at 126.74972 64.046) (size 0.5) (drill 0.3) (layers F.Cu B.Cu) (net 3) (status 30))
 (via (at 124.74972 65.046) (size 0.5) (drill 0.3) (layers F.Cu B.Cu) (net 3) (status 30))
 (via (at 124.74972 63.046) (size 0.5) (drill 0.3) (layers F.Cu B.Cu) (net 3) (status 30))
 (via (at 125.74972 63.046) (size 0.5) (drill 0.3) (layers F.Cu B.Cu) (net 3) (status 30))
 (via (at 126.83 63.1) (size 0.5) (drill 0.3) (layers F.Cu B.Cu) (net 3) (status 30))
 (via (at 124.74972 64.046) (size 0.5) (drill 0.3) (layers F.Cu B.Cu) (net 3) (status 30))
 (via (at 125.7708 64.0092) (size 0.8) (drill 0.4) (layers F.Cu B.Cu) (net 3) (status 30))
 (via (at 126.74972 65.046) (size 0.5) (drill 0.3) (layers F.Cu B.Cu) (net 3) (status 30))
 (via (at 125.74972 65.046) (size 0.5) (drill 0.3) (layers F.Cu B.Cu) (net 3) (status 30))
 (segment (start 122.35 56.38) (end 128.85 56.38) (width 0.5) (layer F.Cu) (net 3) (status 30))
 (segment (start 127.040001 62.230001) (end 126.82 62.01) (width 0.5) (layer B.Cu) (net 3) (status 30))
 (segment (start 130.091999 62.230001) (end 127.040001 62.230001) (width 0.5) (layer B.Cu) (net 3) (status 20))
 (segment (start 131.632 60.69) (end 130.091999 62.230001) (width 0.5) (layer B.Cu) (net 3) (status 10))
 (segment (start 126.82 58.41) (end 126.82 62.01) (width 0.5) (layer B.Cu) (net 3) (status 20))
 (segment (start 128.85 56.38) (end 126.82 58.41) (width 0.5) (layer B.Cu) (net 3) (status 10))
 (segment (start 125.7808 63.0492) (end 126.82 62.01) (width 0.5) (layer B.Cu) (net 3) (status 30))
 (segment (start 125.7808 64.0842) (end 125.7808 63.0492) (width 0.5) (layer B.Cu) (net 3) (status 30))
 (segment (start 128.98 64.17) (end 126.82 62.01) (width 0.5) (layer B.Cu) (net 3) (status 20))
 (segment (start 130.98 64.17) (end 128.98 64.17) (width 0.5) (layer B.Cu) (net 3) (status 10))
 (segment (start 120.661 59.309) (end 118.1 61.87) (width 0.5) (layer B.Cu) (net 3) (status 20))
 (segment (start 124.119 59.309) (end 120.661 59.309) (width 0.5) (layer B.Cu) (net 3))
 (segment (start 126.82 62.01) (end 124.119 59.309) (width 0.5) (layer B.Cu) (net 3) (status 10))
 (segment (start 118.1 62.82) (end 119.32 64.04) (width 0.5) (layer B.Cu) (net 3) (status 20))
 (segment (start 118.1 61.87) (end 118.1 62.82) (width 0.5) (layer B.Cu) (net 3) (status 10))
 (segment (start 133.135003 65.869999) (end 132.330001 65.869999) (width 0.5) (layer B.Cu) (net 14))
 (segment (start 134.099999 64.905003) (end 133.135003 65.869999) (width 0.5) (layer B.Cu) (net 14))
 (segment (start 134.099999 61.778001) (end 134.099999 64.905003) (width 0.5) (layer B.Cu) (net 14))
 (segment (start 132.330001 65.869999) (end 130.98 67.22) (width 0.5) (layer B.Cu) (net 14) (status 20))
 (segment (start 135.188 60.69) (end 134.099999 61.778001) (width 0.5) (layer B.Cu) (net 14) (status 10))
 (segment (start 130.048 76.832) (end 128.72 78.16) (width 0.5) (layer F.Cu) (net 12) (status 20))
 (segment (start 130.048 75.3488) (end 130.048 76.832) (width 0.5) (layer F.Cu) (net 12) (status 10))
 (segment (start 130.58501 66.64) (end 132.85 64.37501) (width 0.5) (layer F.Cu) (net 15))
 (via (at 132.85 64.37501) (size 0.8) (drill 0.4) (layers F.Cu B.Cu) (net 15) (status 30))
 (segment (start 122.9 66.64) (end 130.58501 66.64) (width 0.5) (layer F.Cu) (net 15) (status 10))
 (via (at 122.7836 78.2066) (size 0.5) (drill 0.3) (layers F.Cu B.Cu) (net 10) (status 30))
 (segment (start 122.7836 78.2066) (end 122.7836 68.2036) (width 0.5) (layer B.Cu) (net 10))
 (segment (start 122.7836 68.2036) (end 121.22 66.64) (width 0.5) (layer B.Cu) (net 10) (status 20))
 (via (at 122.7836 68.2036) (size 0.5) (drill 0.3) (layers F.Cu B.Cu) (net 10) (status 30))
 (segment (start 123.0376 69.9499) (end 123.1575 69.83) (width 0.5) (layer F.Cu) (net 17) (status 30))
 (segment (start 123.0376 73.0188) (end 123.0376 69.9499) (width 0.5) (layer F.Cu) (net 17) (status 30))
 (segment (start 123.0376 75.8424) (end 120.72 78.16) (width 0.5) (layer F.Cu) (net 9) (status 30))
 (segment (start 123.0376 75.4188) (end 123.0376 75.8424) (width 0.5) (layer F.Cu) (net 9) (status 30))
 (segment (start 131.41 60.495) (end 131.45 60.535) (width 0.5) (layer F.Cu) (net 18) (status 30))
 (segment (start 131.41 58.52) (end 131.41 60.495) (width 0.5) (layer F.Cu) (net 18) (status 30))
 (via (at 121.33 64.13) (size 0.8) (drill 0.4) (layers F.Cu B.Cu) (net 4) (status 30))
 (segment (start 122.35 63.09) (end 121.31 64.13) (width 0.5) (layer F.Cu) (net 4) (status 20))
 (segment (start 122.35 60.88) (end 122.35 63.09) (width 0.5) (layer F.Cu) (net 4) (status 10))
 (segment (start 122.35 60.88) (end 128.85 60.88) (width 0.5) (layer F.Cu) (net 4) (status 30))
 (segment (start 128.85 58.68) (end 131.41 56.12) (width 0.5) (layer F.Cu) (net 4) (status 20))
 (segment (start 128.85 60.88) (end 128.85 58.68) (width 0.5) (layer F.Cu) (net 4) (status 10))
 (segment (start 131.41 56.12) (end 131.41 56.135) (width 0.5) (layer F.Cu) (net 4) (status 30))
 (via (at 120.21 66.67) (size 0.8) (drill 0.4) (layers F.Cu B.Cu) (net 16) (status 30))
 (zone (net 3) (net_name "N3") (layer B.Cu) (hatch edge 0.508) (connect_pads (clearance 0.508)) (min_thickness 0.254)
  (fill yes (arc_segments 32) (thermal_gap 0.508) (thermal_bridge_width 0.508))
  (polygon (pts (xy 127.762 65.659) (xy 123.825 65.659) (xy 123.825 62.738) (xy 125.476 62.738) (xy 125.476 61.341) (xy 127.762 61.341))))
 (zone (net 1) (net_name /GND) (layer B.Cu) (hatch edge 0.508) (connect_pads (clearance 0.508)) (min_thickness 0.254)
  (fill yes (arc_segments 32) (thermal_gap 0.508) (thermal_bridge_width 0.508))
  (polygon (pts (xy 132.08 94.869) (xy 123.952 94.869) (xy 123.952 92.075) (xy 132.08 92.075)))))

